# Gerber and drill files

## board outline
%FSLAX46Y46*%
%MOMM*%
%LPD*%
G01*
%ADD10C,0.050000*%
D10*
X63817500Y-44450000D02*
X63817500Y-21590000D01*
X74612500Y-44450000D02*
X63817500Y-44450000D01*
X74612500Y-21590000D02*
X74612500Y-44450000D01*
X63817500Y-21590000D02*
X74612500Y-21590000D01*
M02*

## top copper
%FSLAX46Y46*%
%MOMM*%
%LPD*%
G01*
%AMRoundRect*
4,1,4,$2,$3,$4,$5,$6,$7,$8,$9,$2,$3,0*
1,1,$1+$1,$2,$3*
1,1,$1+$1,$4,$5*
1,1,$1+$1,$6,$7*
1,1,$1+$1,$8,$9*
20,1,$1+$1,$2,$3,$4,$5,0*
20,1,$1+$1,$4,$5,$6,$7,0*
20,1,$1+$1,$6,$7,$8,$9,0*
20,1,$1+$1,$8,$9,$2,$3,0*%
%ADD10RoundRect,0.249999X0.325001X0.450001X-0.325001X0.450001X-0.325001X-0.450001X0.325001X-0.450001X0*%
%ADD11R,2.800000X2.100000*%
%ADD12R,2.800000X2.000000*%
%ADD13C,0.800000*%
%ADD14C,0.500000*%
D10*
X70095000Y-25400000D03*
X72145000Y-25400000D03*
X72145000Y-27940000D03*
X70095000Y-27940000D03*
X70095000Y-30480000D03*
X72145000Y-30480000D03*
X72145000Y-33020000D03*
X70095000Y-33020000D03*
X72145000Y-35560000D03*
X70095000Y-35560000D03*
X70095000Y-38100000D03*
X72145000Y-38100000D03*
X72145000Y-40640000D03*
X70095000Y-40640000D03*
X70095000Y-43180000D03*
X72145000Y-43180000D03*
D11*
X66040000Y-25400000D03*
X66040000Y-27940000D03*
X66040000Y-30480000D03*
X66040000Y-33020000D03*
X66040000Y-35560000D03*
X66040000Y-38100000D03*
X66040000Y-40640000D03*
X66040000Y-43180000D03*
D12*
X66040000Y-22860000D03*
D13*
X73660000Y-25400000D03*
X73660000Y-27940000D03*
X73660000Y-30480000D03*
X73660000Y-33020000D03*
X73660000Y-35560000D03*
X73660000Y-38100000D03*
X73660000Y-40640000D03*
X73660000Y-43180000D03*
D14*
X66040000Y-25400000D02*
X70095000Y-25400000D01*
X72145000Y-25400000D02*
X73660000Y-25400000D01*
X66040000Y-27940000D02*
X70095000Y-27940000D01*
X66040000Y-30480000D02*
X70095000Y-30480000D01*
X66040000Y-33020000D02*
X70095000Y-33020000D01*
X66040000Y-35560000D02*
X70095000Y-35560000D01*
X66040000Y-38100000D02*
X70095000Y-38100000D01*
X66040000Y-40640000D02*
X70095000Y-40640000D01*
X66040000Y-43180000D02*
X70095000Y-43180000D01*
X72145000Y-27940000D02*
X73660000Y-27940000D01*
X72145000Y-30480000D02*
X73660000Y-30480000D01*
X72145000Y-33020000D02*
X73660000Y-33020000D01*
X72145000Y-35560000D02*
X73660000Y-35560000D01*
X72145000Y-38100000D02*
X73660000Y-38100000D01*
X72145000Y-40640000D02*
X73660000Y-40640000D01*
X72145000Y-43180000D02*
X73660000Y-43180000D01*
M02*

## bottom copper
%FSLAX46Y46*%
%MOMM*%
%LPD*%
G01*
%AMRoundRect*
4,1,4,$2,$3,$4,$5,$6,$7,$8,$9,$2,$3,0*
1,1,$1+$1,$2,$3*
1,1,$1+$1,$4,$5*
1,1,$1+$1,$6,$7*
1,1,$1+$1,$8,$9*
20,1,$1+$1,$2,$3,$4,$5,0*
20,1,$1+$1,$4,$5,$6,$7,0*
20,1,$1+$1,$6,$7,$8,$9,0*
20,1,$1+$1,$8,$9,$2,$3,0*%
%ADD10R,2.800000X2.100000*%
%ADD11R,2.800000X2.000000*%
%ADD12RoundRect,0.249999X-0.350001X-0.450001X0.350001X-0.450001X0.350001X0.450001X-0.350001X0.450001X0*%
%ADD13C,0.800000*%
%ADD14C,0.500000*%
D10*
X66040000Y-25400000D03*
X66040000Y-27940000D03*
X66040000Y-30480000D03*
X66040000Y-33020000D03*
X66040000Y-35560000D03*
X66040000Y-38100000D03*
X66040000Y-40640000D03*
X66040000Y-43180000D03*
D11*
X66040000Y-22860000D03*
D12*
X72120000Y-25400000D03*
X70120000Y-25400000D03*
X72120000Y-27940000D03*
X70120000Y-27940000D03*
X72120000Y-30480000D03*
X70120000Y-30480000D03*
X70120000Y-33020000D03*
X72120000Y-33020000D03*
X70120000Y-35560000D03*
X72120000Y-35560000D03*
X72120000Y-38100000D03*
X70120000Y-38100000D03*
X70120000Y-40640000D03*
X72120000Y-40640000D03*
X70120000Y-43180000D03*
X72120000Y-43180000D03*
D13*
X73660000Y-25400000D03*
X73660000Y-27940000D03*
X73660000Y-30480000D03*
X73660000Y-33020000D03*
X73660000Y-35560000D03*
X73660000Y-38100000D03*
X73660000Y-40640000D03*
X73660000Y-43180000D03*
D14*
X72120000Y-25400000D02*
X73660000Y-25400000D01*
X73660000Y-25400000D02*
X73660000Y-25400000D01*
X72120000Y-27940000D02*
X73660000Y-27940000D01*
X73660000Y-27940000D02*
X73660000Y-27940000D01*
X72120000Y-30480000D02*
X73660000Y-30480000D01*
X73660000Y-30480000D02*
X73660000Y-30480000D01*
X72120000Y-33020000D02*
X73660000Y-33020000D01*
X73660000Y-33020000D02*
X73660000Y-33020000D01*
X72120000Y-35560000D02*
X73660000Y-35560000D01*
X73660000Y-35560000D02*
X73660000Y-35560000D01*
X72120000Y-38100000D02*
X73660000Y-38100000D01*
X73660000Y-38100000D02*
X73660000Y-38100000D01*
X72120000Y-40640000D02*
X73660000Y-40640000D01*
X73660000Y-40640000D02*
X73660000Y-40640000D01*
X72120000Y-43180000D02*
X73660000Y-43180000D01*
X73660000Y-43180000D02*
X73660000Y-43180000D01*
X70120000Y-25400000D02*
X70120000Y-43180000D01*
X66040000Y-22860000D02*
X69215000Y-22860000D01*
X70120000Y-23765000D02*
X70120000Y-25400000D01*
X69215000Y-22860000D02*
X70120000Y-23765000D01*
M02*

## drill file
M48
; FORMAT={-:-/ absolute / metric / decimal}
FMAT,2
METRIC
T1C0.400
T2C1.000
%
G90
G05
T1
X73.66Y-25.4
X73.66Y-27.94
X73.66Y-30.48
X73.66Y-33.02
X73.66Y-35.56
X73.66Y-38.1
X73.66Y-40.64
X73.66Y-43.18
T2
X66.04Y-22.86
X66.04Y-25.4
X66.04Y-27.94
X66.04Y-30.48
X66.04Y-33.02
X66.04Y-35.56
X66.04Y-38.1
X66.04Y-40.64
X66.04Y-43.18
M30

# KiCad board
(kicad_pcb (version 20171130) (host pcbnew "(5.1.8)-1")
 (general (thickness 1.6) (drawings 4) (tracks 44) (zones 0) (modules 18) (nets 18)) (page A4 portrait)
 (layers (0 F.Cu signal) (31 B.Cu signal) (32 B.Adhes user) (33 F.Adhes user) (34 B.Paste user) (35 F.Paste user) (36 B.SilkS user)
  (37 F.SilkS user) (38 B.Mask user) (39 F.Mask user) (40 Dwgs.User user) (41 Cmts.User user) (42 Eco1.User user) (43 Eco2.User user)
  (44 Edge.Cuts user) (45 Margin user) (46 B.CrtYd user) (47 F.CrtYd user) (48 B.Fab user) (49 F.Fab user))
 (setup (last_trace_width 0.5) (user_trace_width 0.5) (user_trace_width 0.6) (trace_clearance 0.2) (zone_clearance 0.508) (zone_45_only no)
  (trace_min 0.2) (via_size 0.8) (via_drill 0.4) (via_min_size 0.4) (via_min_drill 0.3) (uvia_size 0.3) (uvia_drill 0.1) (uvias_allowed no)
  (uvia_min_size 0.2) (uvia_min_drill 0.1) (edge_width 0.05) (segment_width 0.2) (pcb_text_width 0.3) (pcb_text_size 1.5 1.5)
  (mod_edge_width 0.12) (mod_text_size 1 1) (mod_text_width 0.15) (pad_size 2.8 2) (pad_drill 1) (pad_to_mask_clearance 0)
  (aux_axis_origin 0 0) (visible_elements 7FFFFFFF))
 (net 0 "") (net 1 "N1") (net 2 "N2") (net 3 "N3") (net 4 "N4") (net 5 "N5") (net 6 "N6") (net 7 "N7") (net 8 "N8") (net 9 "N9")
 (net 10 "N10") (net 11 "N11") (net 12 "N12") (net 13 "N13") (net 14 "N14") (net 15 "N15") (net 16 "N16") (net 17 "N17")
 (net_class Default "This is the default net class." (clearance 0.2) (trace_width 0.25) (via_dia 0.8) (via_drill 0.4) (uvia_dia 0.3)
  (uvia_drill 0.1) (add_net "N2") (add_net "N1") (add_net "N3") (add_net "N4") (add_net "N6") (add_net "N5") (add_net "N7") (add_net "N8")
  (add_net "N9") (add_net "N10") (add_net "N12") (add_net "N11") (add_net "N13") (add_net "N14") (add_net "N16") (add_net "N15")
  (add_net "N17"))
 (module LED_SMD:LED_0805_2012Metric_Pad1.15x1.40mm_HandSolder (layer F.Cu) (at 71.12 25.4 180)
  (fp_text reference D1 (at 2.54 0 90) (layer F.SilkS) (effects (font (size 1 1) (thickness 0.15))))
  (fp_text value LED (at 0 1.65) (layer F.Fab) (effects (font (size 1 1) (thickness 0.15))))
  (pad 2 smd roundrect (at 1.025 0 180) (size 1.15 1.4) (layers F.Cu F.Paste F.Mask) (roundrect_rratio 0.2173904347826087) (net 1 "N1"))
  (pad 1 smd roundrect (at -1.025 0 180) (size 1.15 1.4) (layers F.Cu F.Paste F.Mask) (roundrect_rratio 0.2173904347826087) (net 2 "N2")))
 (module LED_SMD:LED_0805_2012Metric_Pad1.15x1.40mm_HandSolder (layer F.Cu) (at 71.12 27.94 180)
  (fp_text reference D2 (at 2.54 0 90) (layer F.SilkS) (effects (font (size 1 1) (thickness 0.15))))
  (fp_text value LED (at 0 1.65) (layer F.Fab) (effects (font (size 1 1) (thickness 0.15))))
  (pad 1 smd roundrect (at -1.025 0 180) (size 1.15 1.4) (layers F.Cu F.Paste F.Mask) (roundrect_rratio 0.2173904347826087) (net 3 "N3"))
  (pad 2 smd roundrect (at 1.025 0 180) (size 1.15 1.4) (layers F.Cu F.Paste F.Mask) (roundrect_rratio 0.2173904347826087) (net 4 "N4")))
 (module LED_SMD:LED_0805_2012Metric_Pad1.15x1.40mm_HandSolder (layer F.Cu) (at 71.12 30.48 180)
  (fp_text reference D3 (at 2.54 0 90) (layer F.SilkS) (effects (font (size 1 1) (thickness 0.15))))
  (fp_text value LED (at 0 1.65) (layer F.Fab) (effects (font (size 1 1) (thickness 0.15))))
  (pad 2 smd roundrect (at 1.025 0 180) (size 1.15 1.4) (layers F.Cu F.Paste F.Mask) (roundrect_rratio 0.2173904347826087) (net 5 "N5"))
  (pad 1 smd roundrect (at -1.025 0 180) (size 1.15 1.4) (layers F.Cu F.Paste F.Mask) (roundrect_rratio 0.2173904347826087) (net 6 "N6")))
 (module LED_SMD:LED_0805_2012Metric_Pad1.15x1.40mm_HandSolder (layer F.Cu) (at 71.12 33.02 180)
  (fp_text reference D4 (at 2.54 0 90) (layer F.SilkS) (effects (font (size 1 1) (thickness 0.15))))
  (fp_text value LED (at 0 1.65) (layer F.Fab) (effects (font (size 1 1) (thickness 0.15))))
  (pad 1 smd roundrect (at -1.025 0 180) (size 1.15 1.4) (layers F.Cu F.Paste F.Mask) (roundrect_rratio 0.2173904347826087) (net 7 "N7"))
  (pad 2 smd roundrect (at 1.025 0 180) (size 1.15 1.4) (layers F.Cu F.Paste F.Mask) (roundrect_rratio 0.2173904347826087) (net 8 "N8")))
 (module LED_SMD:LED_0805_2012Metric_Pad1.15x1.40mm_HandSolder (layer F.Cu) (at 71.12 35.56 180)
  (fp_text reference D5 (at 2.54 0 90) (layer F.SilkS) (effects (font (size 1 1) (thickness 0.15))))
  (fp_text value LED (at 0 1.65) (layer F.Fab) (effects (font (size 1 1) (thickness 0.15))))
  (pad 1 smd roundrect (at -1.025 0 180) (size 1.15 1.4) (layers F.Cu F.Paste F.Mask) (roundrect_rratio 0.2173904347826087) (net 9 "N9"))
  (pad 2 smd roundrect (at 1.025 0 180) (size 1.15 1.4) (layers F.Cu F.Paste F.Mask) (roundrect_rratio 0.2173904347826087) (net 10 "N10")))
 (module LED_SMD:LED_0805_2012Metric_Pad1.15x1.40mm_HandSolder (layer F.Cu) (at 71.12 38.1 180)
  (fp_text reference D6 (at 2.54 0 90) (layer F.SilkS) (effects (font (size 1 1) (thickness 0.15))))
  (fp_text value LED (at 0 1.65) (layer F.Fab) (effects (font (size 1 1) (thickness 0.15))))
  (pad 2 smd roundrect (at 1.025 0 180) (size 1.15 1.4) (layers F.Cu F.Paste F.Mask) (roundrect_rratio 0.2173904347826087) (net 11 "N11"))
  (pad 1 smd roundrect (at -1.025 0 180) (size 1.15 1.4) (layers F.Cu F.Paste F.Mask) (roundrect_rratio 0.2173904347826087) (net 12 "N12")))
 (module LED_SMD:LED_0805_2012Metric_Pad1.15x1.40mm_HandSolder (layer F.Cu) (at 71.12 40.64 180)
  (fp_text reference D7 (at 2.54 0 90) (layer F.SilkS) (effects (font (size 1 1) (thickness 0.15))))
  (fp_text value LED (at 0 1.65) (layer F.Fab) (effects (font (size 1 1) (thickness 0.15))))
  (pad 1 smd roundrect (at -1.025 0 180) (size 1.15 1.4) (layers F.Cu F.Paste F.Mask) (roundrect_rratio 0.2173904347826087) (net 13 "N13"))
  (pad 2 smd roundrect (at 1.025 0 180) (size 1.15 1.4) (layers F.Cu F.Paste F.Mask) (roundrect_rratio 0.2173904347826087) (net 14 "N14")))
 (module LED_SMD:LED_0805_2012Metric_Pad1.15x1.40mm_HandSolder (layer F.Cu) (at 71.12 43.18 180)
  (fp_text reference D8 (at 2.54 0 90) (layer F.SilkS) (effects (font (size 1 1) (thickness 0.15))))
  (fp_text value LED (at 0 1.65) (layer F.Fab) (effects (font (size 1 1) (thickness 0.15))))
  (pad 2 smd roundrect (at 1.025 0 180) (size 1.15 1.4) (layers F.Cu F.Paste F.Mask) (roundrect_rratio 0.2173904347826087) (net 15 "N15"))
  (pad 1 smd roundrect (at -1.025 0 180) (size 1.15 1.4) (layers F.Cu F.Paste F.Mask) (roundrect_rratio 0.2173904347826087) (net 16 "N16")))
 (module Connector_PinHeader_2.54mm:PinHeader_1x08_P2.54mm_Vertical (layer B.Cu) (at 66.04 25.4 180)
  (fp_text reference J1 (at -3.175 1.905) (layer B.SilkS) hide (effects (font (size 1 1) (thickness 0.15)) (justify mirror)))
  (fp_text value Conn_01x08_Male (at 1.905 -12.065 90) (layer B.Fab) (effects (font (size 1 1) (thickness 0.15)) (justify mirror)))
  (pad 1 thru_hole rect (at 0 0 180) (size 2.8 2.1) (drill 1) (layers *.Cu *.Mask) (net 1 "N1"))
  (pad 2 thru_hole rect (at 0 -2.54 180) (size 2.8 2.1) (drill 1) (layers *.Cu *.Mask) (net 4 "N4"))
  (pad 3 thru_hole rect (at 0 -5.08 180) (size 2.8 2.1) (drill 1) (layers *.Cu *.Mask) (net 5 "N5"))
  (pad 4 thru_hole rect (at 0 -7.62 180) (size 2.8 2.1) (drill 1) (layers *.Cu *.Mask) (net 8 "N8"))
  (pad 5 thru_hole rect (at 0 -10.16 180) (size 2.8 2.1) (drill 1) (layers *.Cu *.Mask) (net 10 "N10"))
  (pad 6 thru_hole rect (at 0 -12.7 180) (size 2.8 2.1) (drill 1) (layers *.Cu *.Mask) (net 11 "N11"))
  (pad 7 thru_hole rect (at 0 -15.24 180) (size 2.8 2.1) (drill 1) (layers *.Cu *.Mask) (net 14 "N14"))
  (pad 8 thru_hole rect (at 0 -17.78 180) (size 2.8 2.1) (drill 1) (layers *.Cu *.Mask) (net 15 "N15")))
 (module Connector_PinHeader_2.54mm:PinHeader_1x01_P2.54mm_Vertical (layer B.Cu) (at 66.04 22.86)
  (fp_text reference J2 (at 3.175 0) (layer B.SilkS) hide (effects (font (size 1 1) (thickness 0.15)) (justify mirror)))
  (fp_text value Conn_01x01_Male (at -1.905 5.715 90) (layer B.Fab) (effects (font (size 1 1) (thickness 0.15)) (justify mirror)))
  (pad 1 thru_hole rect (at 0 0) (size 2.8 2) (drill 1) (layers *.Cu *.Mask) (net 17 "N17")))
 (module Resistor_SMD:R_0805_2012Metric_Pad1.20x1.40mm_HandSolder (layer B.Cu) (at 71.12 25.4)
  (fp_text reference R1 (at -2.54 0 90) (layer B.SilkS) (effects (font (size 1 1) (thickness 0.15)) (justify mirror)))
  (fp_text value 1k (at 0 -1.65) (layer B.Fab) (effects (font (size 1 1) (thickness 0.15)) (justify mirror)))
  (pad 2 smd roundrect (at 1 0) (size 1.2 1.4) (layers B.Cu B.Paste B.Mask) (roundrect_rratio 0.2083325) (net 2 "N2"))
  (pad 1 smd roundrect (at -1 0) (size 1.2 1.4) (layers B.Cu B.Paste B.Mask) (roundrect_rratio 0.2083325) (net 17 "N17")))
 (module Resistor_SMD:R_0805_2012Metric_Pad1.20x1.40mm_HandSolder (layer B.Cu) (at 71.12 27.94)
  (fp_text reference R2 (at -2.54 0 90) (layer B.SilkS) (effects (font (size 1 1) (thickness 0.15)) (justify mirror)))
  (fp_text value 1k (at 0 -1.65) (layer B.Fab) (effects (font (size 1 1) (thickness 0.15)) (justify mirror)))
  (pad 2 smd roundrect (at 1 0) (size 1.2 1.4) (layers B.Cu B.Paste B.Mask) (roundrect_rratio 0.2083325) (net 3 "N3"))
  (pad 1 smd roundrect (at -1 0) (size 1.2 1.4) (layers B.Cu B.Paste B.Mask) (roundrect_rratio 0.2083325) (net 17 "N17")))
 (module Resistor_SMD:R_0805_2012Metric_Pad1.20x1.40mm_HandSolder (layer B.Cu) (at 71.12 30.48)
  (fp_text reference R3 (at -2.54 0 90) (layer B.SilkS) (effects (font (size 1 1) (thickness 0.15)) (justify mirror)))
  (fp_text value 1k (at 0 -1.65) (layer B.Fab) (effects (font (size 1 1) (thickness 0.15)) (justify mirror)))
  (pad 2 smd roundrect (at 1 0) (size 1.2 1.4) (layers B.Cu B.Paste B.Mask) (roundrect_rratio 0.2083325) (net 6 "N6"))
  (pad 1 smd roundrect (at -1 0) (size 1.2 1.4) (layers B.Cu B.Paste B.Mask) (roundrect_rratio 0.2083325) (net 17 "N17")))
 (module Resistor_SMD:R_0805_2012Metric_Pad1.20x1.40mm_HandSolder (layer B.Cu) (at 71.12 33.02)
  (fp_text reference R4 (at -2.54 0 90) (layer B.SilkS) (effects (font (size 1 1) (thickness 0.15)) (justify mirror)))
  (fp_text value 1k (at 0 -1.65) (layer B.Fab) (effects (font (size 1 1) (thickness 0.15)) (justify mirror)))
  (pad 1 smd roundrect (at -1 0) (size 1.2 1.4) (layers B.Cu B.Paste B.Mask) (roundrect_rratio 0.2083325) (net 17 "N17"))
  (pad 2 smd roundrect (at 1 0) (size 1.2 1.4) (layers B.Cu B.Paste B.Mask) (roundrect_rratio 0.2083325) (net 7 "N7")))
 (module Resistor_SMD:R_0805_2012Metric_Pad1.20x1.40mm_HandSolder (layer B.Cu) (at 71.12 35.56)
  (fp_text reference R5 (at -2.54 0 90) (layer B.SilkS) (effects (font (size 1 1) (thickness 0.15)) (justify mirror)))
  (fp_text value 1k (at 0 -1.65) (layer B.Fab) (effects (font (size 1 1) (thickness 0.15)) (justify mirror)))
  (pad 1 smd roundrect (at -1 0) (size 1.2 1.4) (layers B.Cu B.Paste B.Mask) (roundrect_rratio 0.2083325) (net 17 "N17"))
  (pad 2 smd roundrect (at 1 0) (size 1.2 1.4) (layers B.Cu B.Paste B.Mask) (roundrect_rratio 0.2083325) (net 9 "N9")))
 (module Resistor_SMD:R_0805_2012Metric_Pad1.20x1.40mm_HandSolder (layer B.Cu) (at 71.12 38.1)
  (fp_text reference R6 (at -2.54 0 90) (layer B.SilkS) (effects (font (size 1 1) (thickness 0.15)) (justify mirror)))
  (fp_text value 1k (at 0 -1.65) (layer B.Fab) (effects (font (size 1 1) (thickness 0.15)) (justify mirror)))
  (pad 2 smd roundrect (at 1 0) (size 1.2 1.4) (layers B.Cu B.Paste B.Mask) (roundrect_rratio 0.2083325) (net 12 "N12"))
  (pad 1 smd roundrect (at -1 0) (size 1.2 1.4) (layers B.Cu B.Paste B.Mask) (roundrect_rratio 0.2083325) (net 17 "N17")))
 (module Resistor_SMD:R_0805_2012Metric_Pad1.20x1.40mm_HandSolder (layer B.Cu) (at 71.12 40.64)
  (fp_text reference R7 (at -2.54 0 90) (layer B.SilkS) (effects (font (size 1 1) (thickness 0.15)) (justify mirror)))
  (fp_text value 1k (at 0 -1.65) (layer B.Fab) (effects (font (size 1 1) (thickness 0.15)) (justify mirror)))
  (pad 1 smd roundrect (at -1 0) (size 1.2 1.4) (layers B.Cu B.Paste B.Mask) (roundrect_rratio 0.2083325) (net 17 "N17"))
  (pad 2 smd roundrect (at 1 0) (size 1.2 1.4) (layers B.Cu B.Paste B.Mask) (roundrect_rratio 0.2083325) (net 13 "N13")))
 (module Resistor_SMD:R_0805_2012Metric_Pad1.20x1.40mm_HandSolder (layer B.Cu) (at 71.12 43.18)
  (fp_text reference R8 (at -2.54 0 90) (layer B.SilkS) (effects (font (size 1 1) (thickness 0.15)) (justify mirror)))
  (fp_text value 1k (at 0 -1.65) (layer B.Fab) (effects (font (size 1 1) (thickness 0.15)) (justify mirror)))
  (pad 1 smd roundrect (at -1 0) (size 1.2 1.4) (layers B.Cu B.Paste B.Mask) (roundrect_rratio 0.2083325) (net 17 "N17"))
  (pad 2 smd roundrect (at 1 0) (size 1.2 1.4) (layers B.Cu B.Paste B.Mask) (roundrect_rratio 0.2083325) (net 16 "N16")))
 (gr_line (start 63.8175 44.45) (end 63.8175 21.59) (layer Edge.Cuts) (width 0.05))
 (gr_line (start 74.6125 44.45) (end 63.8175 44.45) (layer Edge.Cuts) (width 0.05))
 (gr_line (start 74.6125 21.59) (end 74.6125 44.45) (layer Edge.Cuts) (width 0.05))
 (gr_line (start 63.8175 21.59) (end 74.6125 21.59) (layer Edge.Cuts) (width 0.05))
 (segment (start 66.04 25.4) (end 70.095 25.4) (width 0.5) (layer F.Cu) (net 1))
 (segment (start 72.12 25.4) (end 73.66 25.4) (width 0.5) (layer B.Cu) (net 2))
 (segment (start 73.66 25.4) (end 73.66 25.4) (width 0.5) (layer B.Cu) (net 2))
 (via (at 73.66 25.4) (size 0.8) (drill 0.4) (layers F.Cu B.Cu) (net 2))
 (segment (start 72.145 25.4) (end 73.66 25.4) (width 0.5) (layer F.Cu) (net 2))
 (segment (start 66.04 27.94) (end 70.095 27.94) (width 0.5) (layer F.Cu) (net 4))
 (segment (start 66.04 30.48) (end 70.095 30.48) (width 0.5) (layer F.Cu) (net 5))
 (segment (start 66.04 33.02) (end 70.095 33.02) (width 0.5) (layer F.Cu) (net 8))
 (segment (start 66.04 35.56) (end 70.095 35.56) (width 0.5) (layer F.Cu) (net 10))
 (segment (start 66.04 38.1) (end 70.095 38.1) (width 0.5) (layer F.Cu) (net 11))
 (segment (start 66.04 40.64) (end 70.095 40.64) (width 0.5) (layer F.Cu) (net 14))
 (segment (start 66.04 43.18) (end 70.095 43.18) (width 0.5) (layer F.Cu) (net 15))
 (segment (start 72.12 27.94) (end 73.66 27.94) (width 0.5) (layer B.Cu) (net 3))
 (segment (start 73.66 27.94) (end 73.66 27.94) (width 0.5) (layer B.Cu) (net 3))
 (via (at 73.66 27.94) (size 0.8) (drill 0.4) (layers F.Cu B.Cu) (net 3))
 (segment (start 72.145 27.94) (end 73.66 27.94) (width 0.5) (layer F.Cu) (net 3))
 (segment (start 72.12 30.48) (end 73.66 30.48) (width 0.5) (layer B.Cu) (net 6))
 (segment (start 73.66 30.48) (end 73.66 30.48) (width 0.5) (layer B.Cu) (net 6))
 (via (at 73.66 30.48) (size 0.8) (drill 0.4) (layers F.Cu B.Cu) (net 6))
 (segment (start 72.145 30.48) (end 73.66 30.48) (width 0.5) (layer F.Cu) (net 6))
 (segment (start 72.12 33.02) (end 73.66 33.02) (width 0.5) (layer B.Cu) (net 7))
 (segment (start 73.66 33.02) (end 73.66 33.02) (width 0.5) (layer B.Cu) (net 7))
 (via (at 73.66 33.02) (size 0.8) (drill 0.4) (layers F.Cu B.Cu) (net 7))
 (segment (start 72.145 33.02) (end 73.66 33.02) (width 0.5) (layer F.Cu) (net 7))
 (segment (start 72.12 35.56) (end 73.66 35.56) (width 0.5) (layer B.Cu) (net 9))
 (segment (start 73.66 35.56) (end 73.66 35.56) (width 0.5) (layer B.Cu) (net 9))
 (via (at 73.66 35.56) (size 0.8) (drill 0.4) (layers F.Cu B.Cu) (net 9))
 (segment (start 72.145 35.56) (end 73.66 35.56) (width 0.5) (layer F.Cu) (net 9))
 (segment (start 72.12 38.1) (end 73.66 38.1) (width 0.5) (layer B.Cu) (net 12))
 (segment (start 73.66 38.1) (end 73.66 38.1) (width 0.5) (layer B.Cu) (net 12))
 (via (at 73.66 38.1) (size 0.8) (drill 0.4) (layers F.Cu B.Cu) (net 12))
 (segment (start 72.145 38.1) (end 73.66 38.1) (width 0.5) (layer F.Cu) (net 12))
 (segment (start 72.12 40.64) (end 73.66 40.64) (width 0.5) (layer B.Cu) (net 13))
 (segment (start 73.66 40.64) (end 73.66 40.64) (width 0.5) (layer B.Cu) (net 13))
 (via (at 73.66 40.64) (size 0.8) (drill 0.4) (layers F.Cu B.Cu) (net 13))
 (segment (start 72.145 40.64) (end 73.66 40.64) (width 0.5) (layer F.Cu) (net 13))
 (segment (start 72.12 43.18) (end 73.66 43.18) (width 0.5) (layer B.Cu) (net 16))
 (segment (start 73.66 43.18) (end 73.66 43.18) (width 0.5) (layer B.Cu) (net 16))
 (via (at 73.66 43.18) (size 0.8) (drill 0.4) (layers F.Cu B.Cu) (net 16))
 (segment (start 72.145 43.18) (end 73.66 43.18) (width 0.5) (layer F.Cu) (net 16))
 (segment (start 70.12 25.4) (end 70.12 43.18) (width 0.5) (layer B.Cu) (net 17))
 (segment (start 66.04 22.86) (end 69.215 22.86) (width 0.5) (layer B.Cu) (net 17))
 (segment (start 70.12 23.765) (end 70.12 25.4) (width 0.5) (layer B.Cu) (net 17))
 (segment (start 69.215 22.86) (end 70.12 23.765) (width 0.5) (layer B.Cu) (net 17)))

